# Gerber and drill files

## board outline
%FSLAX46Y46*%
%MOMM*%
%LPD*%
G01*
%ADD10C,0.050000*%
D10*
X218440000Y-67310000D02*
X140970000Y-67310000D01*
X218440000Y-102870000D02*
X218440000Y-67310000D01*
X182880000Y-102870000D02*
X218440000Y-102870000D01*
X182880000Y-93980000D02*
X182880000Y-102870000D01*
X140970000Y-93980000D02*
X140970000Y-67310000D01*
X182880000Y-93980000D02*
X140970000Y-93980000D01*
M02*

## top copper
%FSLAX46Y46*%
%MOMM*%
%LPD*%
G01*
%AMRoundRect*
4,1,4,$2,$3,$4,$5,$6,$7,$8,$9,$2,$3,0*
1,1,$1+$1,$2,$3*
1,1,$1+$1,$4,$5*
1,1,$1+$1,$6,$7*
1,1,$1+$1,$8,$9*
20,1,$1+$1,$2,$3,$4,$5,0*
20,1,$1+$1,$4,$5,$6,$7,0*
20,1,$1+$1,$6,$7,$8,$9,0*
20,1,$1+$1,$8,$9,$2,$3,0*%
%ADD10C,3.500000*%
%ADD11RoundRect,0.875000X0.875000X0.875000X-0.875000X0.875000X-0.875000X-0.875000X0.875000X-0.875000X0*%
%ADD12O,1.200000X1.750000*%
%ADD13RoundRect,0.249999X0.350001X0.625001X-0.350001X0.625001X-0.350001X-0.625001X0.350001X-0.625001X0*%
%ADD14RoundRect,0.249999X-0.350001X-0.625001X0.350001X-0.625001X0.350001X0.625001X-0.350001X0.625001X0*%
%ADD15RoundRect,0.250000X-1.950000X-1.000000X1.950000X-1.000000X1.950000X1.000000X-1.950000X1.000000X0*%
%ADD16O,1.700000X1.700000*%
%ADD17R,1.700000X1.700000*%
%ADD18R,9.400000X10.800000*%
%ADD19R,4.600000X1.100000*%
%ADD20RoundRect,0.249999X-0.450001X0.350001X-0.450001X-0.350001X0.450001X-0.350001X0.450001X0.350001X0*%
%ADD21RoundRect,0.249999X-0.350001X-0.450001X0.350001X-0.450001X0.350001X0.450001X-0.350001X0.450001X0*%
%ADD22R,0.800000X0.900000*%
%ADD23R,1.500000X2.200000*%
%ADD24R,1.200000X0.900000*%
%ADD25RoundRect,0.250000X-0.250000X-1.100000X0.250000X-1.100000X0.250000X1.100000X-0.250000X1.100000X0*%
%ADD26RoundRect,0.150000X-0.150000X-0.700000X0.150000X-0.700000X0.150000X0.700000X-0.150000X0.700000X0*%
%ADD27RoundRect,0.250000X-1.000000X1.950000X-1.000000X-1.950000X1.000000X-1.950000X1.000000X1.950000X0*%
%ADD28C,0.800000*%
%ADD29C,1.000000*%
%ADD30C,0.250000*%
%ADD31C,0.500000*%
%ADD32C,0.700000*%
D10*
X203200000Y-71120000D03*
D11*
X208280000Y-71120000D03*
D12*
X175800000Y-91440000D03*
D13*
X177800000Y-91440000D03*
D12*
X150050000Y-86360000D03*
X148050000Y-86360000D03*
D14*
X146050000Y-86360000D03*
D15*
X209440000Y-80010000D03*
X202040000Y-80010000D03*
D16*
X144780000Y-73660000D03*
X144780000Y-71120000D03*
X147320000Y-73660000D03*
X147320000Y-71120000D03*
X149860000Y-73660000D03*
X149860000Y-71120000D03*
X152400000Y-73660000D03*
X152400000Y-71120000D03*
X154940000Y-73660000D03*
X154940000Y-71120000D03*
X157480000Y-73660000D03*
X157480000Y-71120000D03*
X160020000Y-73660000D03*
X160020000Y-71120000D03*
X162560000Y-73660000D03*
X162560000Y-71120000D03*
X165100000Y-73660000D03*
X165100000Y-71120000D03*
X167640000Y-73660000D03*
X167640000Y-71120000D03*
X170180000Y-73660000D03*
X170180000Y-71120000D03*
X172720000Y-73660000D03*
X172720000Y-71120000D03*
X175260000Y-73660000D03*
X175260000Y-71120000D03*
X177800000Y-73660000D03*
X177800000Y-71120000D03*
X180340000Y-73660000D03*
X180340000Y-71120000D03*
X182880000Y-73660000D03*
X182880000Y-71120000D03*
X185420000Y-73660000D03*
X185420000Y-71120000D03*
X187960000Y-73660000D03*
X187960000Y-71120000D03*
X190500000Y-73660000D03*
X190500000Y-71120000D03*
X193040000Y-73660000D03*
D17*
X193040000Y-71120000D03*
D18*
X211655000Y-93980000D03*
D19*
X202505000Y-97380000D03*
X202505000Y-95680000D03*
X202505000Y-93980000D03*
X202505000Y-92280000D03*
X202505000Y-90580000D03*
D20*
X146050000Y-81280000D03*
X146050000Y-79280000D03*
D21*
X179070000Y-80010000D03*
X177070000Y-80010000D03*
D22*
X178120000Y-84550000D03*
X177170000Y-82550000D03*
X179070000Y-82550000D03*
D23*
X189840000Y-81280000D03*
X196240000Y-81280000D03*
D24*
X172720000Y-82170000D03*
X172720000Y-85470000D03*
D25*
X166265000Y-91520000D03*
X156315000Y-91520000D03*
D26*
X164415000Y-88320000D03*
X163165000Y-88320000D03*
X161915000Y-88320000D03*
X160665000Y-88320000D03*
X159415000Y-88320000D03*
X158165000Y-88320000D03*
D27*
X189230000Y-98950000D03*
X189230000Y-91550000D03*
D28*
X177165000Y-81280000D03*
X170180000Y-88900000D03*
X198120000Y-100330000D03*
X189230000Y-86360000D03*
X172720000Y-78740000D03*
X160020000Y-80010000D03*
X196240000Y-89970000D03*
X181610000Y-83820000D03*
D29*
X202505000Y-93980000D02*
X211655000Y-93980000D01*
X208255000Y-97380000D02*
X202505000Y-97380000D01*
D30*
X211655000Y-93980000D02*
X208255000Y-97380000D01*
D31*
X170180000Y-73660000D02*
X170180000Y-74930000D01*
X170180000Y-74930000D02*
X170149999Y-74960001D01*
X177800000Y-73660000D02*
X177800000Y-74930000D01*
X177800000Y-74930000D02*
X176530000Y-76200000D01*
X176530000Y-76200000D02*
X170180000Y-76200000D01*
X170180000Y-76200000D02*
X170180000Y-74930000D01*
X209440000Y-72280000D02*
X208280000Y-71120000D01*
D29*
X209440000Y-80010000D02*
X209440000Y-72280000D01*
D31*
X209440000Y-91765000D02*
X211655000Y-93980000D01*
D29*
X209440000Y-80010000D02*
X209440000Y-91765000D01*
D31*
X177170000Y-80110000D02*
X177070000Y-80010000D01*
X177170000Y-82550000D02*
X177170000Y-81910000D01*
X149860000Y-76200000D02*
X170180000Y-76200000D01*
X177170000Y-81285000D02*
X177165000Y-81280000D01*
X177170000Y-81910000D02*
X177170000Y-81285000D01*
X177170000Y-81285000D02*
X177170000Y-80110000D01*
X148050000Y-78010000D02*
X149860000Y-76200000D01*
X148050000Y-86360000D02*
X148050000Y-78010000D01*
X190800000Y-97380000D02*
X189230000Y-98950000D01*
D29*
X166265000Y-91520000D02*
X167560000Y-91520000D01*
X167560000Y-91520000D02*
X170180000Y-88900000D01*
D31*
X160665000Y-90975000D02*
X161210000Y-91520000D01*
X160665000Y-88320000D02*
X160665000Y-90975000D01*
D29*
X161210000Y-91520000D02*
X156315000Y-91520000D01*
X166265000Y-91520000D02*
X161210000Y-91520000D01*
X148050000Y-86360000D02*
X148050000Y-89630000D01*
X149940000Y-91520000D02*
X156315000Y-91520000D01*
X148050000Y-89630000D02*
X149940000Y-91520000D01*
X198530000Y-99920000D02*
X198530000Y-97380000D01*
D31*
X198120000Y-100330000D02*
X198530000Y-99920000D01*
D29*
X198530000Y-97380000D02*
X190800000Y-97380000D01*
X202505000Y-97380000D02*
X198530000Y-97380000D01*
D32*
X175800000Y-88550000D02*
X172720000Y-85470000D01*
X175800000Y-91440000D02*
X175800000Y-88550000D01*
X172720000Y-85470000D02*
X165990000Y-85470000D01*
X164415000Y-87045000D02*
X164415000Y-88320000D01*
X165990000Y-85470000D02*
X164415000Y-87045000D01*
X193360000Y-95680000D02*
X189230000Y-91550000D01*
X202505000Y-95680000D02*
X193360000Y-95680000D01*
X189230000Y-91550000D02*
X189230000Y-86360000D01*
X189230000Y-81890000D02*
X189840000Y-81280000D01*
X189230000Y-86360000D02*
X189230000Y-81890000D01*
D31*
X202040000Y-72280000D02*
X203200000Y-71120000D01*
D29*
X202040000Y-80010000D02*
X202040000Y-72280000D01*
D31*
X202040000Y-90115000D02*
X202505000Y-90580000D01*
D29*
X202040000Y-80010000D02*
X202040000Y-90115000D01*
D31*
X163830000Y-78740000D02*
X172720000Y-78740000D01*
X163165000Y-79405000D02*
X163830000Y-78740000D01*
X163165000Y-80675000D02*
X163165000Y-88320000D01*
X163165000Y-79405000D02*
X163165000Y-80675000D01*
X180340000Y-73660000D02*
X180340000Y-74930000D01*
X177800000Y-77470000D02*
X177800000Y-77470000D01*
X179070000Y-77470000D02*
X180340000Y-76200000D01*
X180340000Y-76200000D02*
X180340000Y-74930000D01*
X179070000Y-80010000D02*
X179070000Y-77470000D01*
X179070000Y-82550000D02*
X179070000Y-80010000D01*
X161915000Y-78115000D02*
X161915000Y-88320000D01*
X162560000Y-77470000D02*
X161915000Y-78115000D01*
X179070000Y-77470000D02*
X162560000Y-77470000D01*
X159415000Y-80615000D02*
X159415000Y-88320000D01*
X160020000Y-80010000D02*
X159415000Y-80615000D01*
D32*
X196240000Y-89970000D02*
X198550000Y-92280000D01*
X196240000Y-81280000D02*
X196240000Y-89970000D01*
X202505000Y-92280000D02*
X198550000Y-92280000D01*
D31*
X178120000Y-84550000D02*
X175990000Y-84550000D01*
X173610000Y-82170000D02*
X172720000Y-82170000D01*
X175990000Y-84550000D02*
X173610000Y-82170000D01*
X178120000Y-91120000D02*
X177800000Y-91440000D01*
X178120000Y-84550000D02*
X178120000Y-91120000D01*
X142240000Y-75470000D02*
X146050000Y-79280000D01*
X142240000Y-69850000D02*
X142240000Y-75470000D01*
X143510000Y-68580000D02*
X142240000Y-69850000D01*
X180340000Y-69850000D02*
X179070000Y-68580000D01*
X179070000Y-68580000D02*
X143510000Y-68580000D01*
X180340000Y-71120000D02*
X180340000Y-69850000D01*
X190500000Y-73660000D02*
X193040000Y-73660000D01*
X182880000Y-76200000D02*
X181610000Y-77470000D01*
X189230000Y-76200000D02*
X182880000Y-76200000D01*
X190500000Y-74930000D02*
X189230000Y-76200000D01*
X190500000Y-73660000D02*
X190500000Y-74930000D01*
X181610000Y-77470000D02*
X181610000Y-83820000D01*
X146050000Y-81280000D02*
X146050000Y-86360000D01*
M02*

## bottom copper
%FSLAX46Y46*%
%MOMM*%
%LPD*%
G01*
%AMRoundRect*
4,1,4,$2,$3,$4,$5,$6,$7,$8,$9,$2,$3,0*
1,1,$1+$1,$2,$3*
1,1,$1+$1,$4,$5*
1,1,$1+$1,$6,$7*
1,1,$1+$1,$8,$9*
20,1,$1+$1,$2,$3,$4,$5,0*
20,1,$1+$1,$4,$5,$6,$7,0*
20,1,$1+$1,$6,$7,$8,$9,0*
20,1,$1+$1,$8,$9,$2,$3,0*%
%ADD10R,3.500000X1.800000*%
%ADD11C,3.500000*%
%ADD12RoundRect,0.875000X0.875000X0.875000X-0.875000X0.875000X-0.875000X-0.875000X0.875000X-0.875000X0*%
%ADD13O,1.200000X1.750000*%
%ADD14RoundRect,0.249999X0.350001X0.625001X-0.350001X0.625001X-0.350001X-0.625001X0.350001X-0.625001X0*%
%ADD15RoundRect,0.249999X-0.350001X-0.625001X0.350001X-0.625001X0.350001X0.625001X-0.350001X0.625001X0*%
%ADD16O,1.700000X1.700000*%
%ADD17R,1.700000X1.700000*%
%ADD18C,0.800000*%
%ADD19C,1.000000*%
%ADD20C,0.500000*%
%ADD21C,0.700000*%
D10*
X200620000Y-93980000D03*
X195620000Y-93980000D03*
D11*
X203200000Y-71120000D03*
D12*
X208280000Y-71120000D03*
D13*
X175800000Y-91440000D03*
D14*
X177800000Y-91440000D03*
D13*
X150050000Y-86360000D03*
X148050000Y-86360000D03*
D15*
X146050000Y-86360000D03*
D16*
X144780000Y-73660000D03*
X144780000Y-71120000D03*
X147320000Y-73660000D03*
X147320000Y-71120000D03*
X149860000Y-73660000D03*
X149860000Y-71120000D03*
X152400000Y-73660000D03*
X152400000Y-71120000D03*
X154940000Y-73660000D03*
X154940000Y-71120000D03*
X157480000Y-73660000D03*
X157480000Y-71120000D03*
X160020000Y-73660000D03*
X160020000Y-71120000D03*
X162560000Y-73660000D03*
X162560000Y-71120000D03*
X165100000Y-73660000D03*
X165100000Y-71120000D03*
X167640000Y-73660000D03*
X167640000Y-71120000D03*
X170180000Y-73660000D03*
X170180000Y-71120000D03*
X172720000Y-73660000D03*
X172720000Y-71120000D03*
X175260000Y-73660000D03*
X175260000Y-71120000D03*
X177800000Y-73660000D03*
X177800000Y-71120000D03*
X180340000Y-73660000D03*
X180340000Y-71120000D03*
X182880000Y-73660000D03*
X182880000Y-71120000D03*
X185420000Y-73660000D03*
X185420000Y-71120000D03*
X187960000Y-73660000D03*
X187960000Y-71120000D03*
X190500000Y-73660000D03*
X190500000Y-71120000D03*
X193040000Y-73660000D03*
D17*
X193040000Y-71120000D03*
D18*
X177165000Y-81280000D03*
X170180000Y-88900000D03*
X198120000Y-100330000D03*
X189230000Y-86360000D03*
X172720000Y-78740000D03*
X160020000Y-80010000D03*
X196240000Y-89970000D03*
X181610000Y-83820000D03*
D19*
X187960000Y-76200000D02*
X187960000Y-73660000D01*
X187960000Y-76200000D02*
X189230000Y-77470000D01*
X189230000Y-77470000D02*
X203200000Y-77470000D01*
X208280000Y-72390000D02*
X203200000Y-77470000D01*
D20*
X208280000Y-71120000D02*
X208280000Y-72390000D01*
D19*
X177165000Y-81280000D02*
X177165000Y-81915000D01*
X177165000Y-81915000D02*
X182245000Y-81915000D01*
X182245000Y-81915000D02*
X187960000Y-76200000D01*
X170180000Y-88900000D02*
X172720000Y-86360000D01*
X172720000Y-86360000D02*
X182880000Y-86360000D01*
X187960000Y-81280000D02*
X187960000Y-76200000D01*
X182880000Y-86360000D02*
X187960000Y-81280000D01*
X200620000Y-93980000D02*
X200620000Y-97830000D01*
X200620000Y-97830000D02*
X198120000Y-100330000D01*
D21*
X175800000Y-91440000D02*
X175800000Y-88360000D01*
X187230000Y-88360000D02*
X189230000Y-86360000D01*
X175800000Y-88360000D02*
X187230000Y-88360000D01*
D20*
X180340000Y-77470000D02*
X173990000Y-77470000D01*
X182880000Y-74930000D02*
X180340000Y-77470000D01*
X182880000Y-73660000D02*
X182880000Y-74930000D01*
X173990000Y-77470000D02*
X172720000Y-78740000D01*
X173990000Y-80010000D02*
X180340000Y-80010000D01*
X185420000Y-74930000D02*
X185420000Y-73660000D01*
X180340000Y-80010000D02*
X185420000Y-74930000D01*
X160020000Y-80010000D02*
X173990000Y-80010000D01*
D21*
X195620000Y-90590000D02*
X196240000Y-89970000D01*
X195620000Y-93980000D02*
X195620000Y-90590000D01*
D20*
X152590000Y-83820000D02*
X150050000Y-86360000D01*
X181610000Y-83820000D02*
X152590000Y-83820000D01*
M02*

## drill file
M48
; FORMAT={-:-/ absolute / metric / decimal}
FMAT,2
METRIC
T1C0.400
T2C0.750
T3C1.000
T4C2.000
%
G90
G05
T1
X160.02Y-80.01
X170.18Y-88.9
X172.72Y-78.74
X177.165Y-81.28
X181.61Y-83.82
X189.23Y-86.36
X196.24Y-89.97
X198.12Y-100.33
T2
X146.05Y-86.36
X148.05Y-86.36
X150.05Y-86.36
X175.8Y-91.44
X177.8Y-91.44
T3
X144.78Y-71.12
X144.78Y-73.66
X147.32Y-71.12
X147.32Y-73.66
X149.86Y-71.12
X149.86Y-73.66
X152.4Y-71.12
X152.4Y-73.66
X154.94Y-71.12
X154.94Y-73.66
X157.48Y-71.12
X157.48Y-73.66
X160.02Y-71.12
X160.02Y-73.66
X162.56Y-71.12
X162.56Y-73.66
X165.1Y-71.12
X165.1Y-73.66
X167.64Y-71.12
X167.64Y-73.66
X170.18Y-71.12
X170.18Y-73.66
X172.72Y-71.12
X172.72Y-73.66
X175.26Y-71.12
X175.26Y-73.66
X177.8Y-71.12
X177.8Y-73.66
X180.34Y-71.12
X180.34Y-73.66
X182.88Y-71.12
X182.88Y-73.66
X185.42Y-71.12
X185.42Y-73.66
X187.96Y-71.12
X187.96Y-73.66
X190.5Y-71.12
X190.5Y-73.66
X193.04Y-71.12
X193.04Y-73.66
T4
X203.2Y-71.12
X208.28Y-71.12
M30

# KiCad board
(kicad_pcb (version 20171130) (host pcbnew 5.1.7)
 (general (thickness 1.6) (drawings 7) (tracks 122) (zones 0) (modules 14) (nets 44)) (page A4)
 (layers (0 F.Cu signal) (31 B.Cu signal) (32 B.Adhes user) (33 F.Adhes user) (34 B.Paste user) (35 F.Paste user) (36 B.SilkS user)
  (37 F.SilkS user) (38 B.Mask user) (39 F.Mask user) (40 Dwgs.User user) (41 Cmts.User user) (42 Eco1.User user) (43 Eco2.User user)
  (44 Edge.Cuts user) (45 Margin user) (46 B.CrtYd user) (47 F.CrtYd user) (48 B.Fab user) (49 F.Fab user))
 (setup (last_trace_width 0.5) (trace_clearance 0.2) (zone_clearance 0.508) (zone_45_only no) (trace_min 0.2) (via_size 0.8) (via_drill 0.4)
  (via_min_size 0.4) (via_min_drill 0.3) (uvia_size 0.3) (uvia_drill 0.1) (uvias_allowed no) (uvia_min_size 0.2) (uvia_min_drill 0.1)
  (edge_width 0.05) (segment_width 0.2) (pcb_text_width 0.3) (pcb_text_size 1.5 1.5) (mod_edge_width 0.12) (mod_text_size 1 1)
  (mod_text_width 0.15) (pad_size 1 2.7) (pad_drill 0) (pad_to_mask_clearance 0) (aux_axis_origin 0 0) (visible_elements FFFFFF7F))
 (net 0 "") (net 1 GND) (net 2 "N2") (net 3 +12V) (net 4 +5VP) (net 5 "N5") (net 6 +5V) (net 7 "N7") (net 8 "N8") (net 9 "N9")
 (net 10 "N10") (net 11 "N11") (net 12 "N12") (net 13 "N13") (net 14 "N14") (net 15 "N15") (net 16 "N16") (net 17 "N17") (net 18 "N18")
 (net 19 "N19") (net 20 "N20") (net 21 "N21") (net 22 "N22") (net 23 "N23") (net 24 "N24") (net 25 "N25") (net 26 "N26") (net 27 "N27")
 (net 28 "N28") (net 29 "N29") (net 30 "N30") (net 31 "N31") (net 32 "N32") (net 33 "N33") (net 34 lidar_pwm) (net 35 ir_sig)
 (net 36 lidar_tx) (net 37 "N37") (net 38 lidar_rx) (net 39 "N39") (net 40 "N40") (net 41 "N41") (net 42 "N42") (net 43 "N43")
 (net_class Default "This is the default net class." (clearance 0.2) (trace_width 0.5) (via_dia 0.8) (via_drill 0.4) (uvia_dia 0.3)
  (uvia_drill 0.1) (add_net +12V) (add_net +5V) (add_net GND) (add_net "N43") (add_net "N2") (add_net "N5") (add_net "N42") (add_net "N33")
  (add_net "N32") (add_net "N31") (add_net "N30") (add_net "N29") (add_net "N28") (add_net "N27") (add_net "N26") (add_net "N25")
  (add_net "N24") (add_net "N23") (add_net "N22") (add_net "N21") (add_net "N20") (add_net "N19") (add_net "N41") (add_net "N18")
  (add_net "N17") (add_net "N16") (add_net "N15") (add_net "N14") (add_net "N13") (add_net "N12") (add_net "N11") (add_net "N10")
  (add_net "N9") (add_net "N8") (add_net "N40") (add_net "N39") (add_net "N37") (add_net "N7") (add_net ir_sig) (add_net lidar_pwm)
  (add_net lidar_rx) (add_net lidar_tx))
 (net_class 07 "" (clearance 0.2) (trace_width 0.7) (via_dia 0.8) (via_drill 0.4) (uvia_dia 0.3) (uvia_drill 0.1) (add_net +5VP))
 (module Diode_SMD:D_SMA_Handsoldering (layer B.Cu) (at 198.12 93.98)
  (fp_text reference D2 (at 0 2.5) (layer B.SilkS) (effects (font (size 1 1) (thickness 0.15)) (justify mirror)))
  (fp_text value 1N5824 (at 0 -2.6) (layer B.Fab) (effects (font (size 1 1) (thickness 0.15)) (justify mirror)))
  (pad 2 smd rect (at 2.5 0) (size 3.5 1.8) (layers B.Cu B.Paste B.Mask) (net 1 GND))
  (pad 1 smd rect (at -2.5 0) (size 3.5 1.8) (layers B.Cu B.Paste B.Mask) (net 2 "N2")))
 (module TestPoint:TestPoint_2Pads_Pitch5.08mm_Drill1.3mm (layer F.Cu) (at 208.28 71.12 180)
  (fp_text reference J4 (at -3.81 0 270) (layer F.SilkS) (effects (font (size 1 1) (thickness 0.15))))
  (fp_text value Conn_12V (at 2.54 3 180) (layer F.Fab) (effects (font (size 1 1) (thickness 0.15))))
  (pad 2 thru_hole circle (at 5.08 0 180) (size 3.5 3.5) (drill 2) (layers *.Cu *.Mask) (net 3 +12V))
  (pad 1 thru_hole roundrect (at 0 0 180) (size 3.5 3.5) (drill 2) (layers *.Cu *.Mask) (roundrect_rratio 0.25) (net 1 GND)))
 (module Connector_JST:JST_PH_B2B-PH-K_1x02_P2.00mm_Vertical (layer F.Cu) (at 177.8 91.44 180)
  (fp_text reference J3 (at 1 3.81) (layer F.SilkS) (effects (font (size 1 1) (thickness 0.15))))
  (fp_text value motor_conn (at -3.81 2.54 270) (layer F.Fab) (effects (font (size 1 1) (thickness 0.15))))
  (pad 2 thru_hole oval (at 2 0 180) (size 1.2 1.75) (drill 0.75) (layers *.Cu *.Mask) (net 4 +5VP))
  (pad 1 thru_hole roundrect (at 0 0 180) (size 1.2 1.75) (drill 0.75) (layers *.Cu *.Mask) (roundrect_rratio 0.2083325) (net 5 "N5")))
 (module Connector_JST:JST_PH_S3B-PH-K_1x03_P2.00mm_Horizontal (layer F.Cu) (at 146.05 86.36)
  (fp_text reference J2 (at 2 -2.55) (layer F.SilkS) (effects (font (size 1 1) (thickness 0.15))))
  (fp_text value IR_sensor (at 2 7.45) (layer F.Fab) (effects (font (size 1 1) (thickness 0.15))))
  (pad 3 thru_hole oval (at 4 0) (size 1.2 1.75) (drill 0.75) (layers *.Cu *.Mask) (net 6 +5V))
  (pad 2 thru_hole oval (at 2 0) (size 1.2 1.75) (drill 0.75) (layers *.Cu *.Mask) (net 1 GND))
  (pad 1 thru_hole roundrect (at 0 0) (size 1.2 1.75) (drill 0.75) (layers *.Cu *.Mask) (roundrect_rratio 0.2083325) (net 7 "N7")))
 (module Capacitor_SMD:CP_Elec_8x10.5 (layer F.Cu) (at 205.74 80.01)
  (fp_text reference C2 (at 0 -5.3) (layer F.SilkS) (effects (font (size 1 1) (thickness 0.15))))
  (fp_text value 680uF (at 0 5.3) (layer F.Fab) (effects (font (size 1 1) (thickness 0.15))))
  (pad 2 smd roundrect (at 3.7 0) (size 4.4 2.5) (layers F.Cu F.Paste F.Mask) (roundrect_rratio 0.1) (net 1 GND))
  (pad 1 smd roundrect (at -3.7 0) (size 4.4 2.5) (layers F.Cu F.Paste F.Mask) (roundrect_rratio 0.1) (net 3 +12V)))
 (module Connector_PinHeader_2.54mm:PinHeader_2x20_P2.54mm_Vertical (layer F.Cu) (at 193.04 71.12 270)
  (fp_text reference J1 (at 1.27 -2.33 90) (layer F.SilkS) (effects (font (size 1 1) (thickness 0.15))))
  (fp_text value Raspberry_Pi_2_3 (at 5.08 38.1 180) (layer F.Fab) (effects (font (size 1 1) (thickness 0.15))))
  (pad 40 thru_hole oval (at 2.54 48.26 270) (size 1.7 1.7) (drill 1) (layers *.Cu *.Mask) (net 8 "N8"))
  (pad 39 thru_hole oval (at 0 48.26 270) (size 1.7 1.7) (drill 1) (layers *.Cu *.Mask) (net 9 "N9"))
  (pad 38 thru_hole oval (at 2.54 45.72 270) (size 1.7 1.7) (drill 1) (layers *.Cu *.Mask) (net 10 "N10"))
  (pad 37 thru_hole oval (at 0 45.72 270) (size 1.7 1.7) (drill 1) (layers *.Cu *.Mask) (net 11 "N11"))
  (pad 36 thru_hole oval (at 2.54 43.18 270) (size 1.7 1.7) (drill 1) (layers *.Cu *.Mask) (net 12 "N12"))
  (pad 35 thru_hole oval (at 0 43.18 270) (size 1.7 1.7) (drill 1) (layers *.Cu *.Mask) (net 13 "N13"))
  (pad 34 thru_hole oval (at 2.54 40.64 270) (size 1.7 1.7) (drill 1) (layers *.Cu *.Mask) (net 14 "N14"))
  (pad 33 thru_hole oval (at 0 40.64 270) (size 1.7 1.7) (drill 1) (layers *.Cu *.Mask) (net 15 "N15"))
  (pad 32 thru_hole oval (at 2.54 38.1 270) (size 1.7 1.7) (drill 1) (layers *.Cu *.Mask) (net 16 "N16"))
  (pad 31 thru_hole oval (at 0 38.1 270) (size 1.7 1.7) (drill 1) (layers *.Cu *.Mask) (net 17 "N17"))
  (pad 30 thru_hole oval (at 2.54 35.56 270) (size 1.7 1.7) (drill 1) (layers *.Cu *.Mask) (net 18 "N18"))
  (pad 29 thru_hole oval (at 0 35.56 270) (size 1.7 1.7) (drill 1) (layers *.Cu *.Mask) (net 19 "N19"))
  (pad 28 thru_hole oval (at 2.54 33.02 270) (size 1.7 1.7) (drill 1) (layers *.Cu *.Mask) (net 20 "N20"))
  (pad 27 thru_hole oval (at 0 33.02 270) (size 1.7 1.7) (drill 1) (layers *.Cu *.Mask) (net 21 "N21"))
  (pad 26 thru_hole oval (at 2.54 30.48 270) (size 1.7 1.7) (drill 1) (layers *.Cu *.Mask) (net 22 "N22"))
  (pad 25 thru_hole oval (at 0 30.48 270) (size 1.7 1.7) (drill 1) (layers *.Cu *.Mask) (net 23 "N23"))
  (pad 24 thru_hole oval (at 2.54 27.94 270) (size 1.7 1.7) (drill 1) (layers *.Cu *.Mask) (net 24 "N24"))
  (pad 23 thru_hole oval (at 0 27.94 270) (size 1.7 1.7) (drill 1) (layers *.Cu *.Mask) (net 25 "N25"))
  (pad 22 thru_hole oval (at 2.54 25.4 270) (size 1.7 1.7) (drill 1) (layers *.Cu *.Mask) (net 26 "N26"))
  (pad 21 thru_hole oval (at 0 25.4 270) (size 1.7 1.7) (drill 1) (layers *.Cu *.Mask) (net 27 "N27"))
  (pad 20 thru_hole oval (at 2.54 22.86 270) (size 1.7 1.7) (drill 1) (layers *.Cu *.Mask) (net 1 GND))
  (pad 19 thru_hole oval (at 0 22.86 270) (size 1.7 1.7) (drill 1) (layers *.Cu *.Mask) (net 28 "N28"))
  (pad 18 thru_hole oval (at 2.54 20.32 270) (size 1.7 1.7) (drill 1) (layers *.Cu *.Mask) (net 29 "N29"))
  (pad 17 thru_hole oval (at 0 20.32 270) (size 1.7 1.7) (drill 1) (layers *.Cu *.Mask) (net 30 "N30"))
  (pad 16 thru_hole oval (at 2.54 17.78 270) (size 1.7 1.7) (drill 1) (layers *.Cu *.Mask) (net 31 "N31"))
  (pad 15 thru_hole oval (at 0 17.78 270) (size 1.7 1.7) (drill 1) (layers *.Cu *.Mask) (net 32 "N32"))
  (pad 14 thru_hole oval (at 2.54 15.24 270) (size 1.7 1.7) (drill 1) (layers *.Cu *.Mask) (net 1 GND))
  (pad 13 thru_hole oval (at 0 15.24 270) (size 1.7 1.7) (drill 1) (layers *.Cu *.Mask) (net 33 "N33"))
  (pad 12 thru_hole oval (at 2.54 12.7 270) (size 1.7 1.7) (drill 1) (layers *.Cu *.Mask) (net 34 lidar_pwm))
  (pad 11 thru_hole oval (at 0 12.7 270) (size 1.7 1.7) (drill 1) (layers *.Cu *.Mask) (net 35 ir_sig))
  (pad 10 thru_hole oval (at 2.54 10.16 270) (size 1.7 1.7) (drill 1) (layers *.Cu *.Mask) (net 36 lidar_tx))
  (pad 9 thru_hole oval (at 0 10.16 270) (size 1.7 1.7) (drill 1) (layers *.Cu *.Mask) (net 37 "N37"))
  (pad 8 thru_hole oval (at 2.54 7.62 270) (size 1.7 1.7) (drill 1) (layers *.Cu *.Mask) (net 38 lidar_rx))
  (pad 7 thru_hole oval (at 0 7.62 270) (size 1.7 1.7) (drill 1) (layers *.Cu *.Mask) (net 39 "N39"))
  (pad 6 thru_hole oval (at 2.54 5.08 270) (size 1.7 1.7) (drill 1) (layers *.Cu *.Mask) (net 1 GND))
  (pad 5 thru_hole oval (at 0 5.08 270) (size 1.7 1.7) (drill 1) (layers *.Cu *.Mask) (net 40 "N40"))
  (pad 4 thru_hole oval (at 2.54 2.54 270) (size 1.7 1.7) (drill 1) (layers *.Cu *.Mask) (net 6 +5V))
  (pad 3 thru_hole oval (at 0 2.54 270) (size 1.7 1.7) (drill 1) (layers *.Cu *.Mask) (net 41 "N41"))
  (pad 2 thru_hole oval (at 2.54 0 270) (size 1.7 1.7) (drill 1) (layers *.Cu *.Mask) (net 6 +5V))
  (pad 1 thru_hole rect (at 0 0 270) (size 1.7 1.7) (drill 1) (layers *.Cu *.Mask) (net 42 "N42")))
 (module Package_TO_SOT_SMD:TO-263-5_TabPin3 (layer F.Cu) (at 208.28 93.98)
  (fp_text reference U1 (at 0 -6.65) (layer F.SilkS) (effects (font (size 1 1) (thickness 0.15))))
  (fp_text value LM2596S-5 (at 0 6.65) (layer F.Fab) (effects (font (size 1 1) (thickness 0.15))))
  (pad "" smd rect (at 0.95 2.775) (size 4.55 5.25) (layers F.Paste))
  (pad "" smd rect (at 5.8 -2.775) (size 4.55 5.25) (layers F.Paste))
  (pad "" smd rect (at 0.95 -2.775) (size 4.55 5.25) (layers F.Paste))
  (pad "" smd rect (at 5.8 2.775) (size 4.55 5.25) (layers F.Paste))
  (pad 3 smd rect (at 3.375 0) (size 9.4 10.8) (layers F.Cu F.Mask) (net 1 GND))
  (pad 5 smd rect (at -5.775 3.4) (size 4.6 1.1) (layers F.Cu F.Paste F.Mask) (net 1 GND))
  (pad 4 smd rect (at -5.775 1.7) (size 4.6 1.1) (layers F.Cu F.Paste F.Mask) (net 4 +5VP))
  (pad 3 smd rect (at -5.775 0) (size 4.6 1.1) (layers F.Cu F.Paste F.Mask) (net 1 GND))
  (pad 2 smd rect (at -5.775 -1.7) (size 4.6 1.1) (layers F.Cu F.Paste F.Mask) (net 2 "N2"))
  (pad 1 smd rect (at -5.775 -3.4) (size 4.6 1.1) (layers F.Cu F.Paste F.Mask) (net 3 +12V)))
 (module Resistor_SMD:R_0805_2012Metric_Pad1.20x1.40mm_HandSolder (layer F.Cu) (at 146.05 80.28 270)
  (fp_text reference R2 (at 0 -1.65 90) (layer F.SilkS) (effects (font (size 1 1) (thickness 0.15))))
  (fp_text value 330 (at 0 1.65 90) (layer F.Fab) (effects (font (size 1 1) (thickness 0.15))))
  (pad 2 smd roundrect (at 1 0 270) (size 1.2 1.4) (layers F.Cu F.Paste F.Mask) (roundrect_rratio 0.2083325) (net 7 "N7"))
  (pad 1 smd roundrect (at -1 0 270) (size 1.2 1.4) (layers F.Cu F.Paste F.Mask) (roundrect_rratio 0.2083325) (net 35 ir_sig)))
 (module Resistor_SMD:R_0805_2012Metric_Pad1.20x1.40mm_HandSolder (layer F.Cu) (at 178.07 80.01)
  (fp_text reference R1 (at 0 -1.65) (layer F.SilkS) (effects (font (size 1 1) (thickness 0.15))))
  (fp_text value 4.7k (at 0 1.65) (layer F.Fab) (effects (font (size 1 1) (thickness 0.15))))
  (pad 2 smd roundrect (at 1 0) (size 1.2 1.4) (layers F.Cu F.Paste F.Mask) (roundrect_rratio 0.2083325) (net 34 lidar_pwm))
  (pad 1 smd roundrect (at -1 0) (size 1.2 1.4) (layers F.Cu F.Paste F.Mask) (roundrect_rratio 0.2083325) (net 1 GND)))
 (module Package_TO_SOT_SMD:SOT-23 (layer F.Cu) (at 178.12 83.55 270)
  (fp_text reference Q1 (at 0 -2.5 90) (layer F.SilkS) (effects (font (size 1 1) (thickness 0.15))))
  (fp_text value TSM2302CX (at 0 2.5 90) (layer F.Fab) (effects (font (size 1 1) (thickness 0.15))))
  (pad 3 smd rect (at 1 0 270) (size 0.9 0.8) (layers F.Cu F.Paste F.Mask) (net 5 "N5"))
  (pad 2 smd rect (at -1 0.95 270) (size 0.9 0.8) (layers F.Cu F.Paste F.Mask) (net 1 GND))
  (pad 1 smd rect (at -1 -0.95 270) (size 0.9 0.8) (layers F.Cu F.Paste F.Mask) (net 34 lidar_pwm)))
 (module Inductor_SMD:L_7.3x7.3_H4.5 (layer F.Cu) (at 193.04 81.28 180)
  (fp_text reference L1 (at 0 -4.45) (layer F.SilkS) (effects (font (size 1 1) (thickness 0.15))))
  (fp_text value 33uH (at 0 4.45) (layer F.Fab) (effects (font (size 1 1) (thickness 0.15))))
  (pad 2 smd rect (at 3.2 0 180) (size 1.5 2.2) (layers F.Cu F.Paste F.Mask) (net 4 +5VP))
  (pad 1 smd rect (at -3.2 0 180) (size 1.5 2.2) (layers F.Cu F.Paste F.Mask) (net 2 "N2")))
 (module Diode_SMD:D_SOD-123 (layer F.Cu) (at 172.72 83.82 90)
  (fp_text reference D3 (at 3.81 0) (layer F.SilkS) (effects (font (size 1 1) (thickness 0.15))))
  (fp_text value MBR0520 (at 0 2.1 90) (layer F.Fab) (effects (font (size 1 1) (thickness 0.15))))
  (pad 2 smd rect (at 1.65 0 90) (size 0.9 1.2) (layers F.Cu F.Paste F.Mask) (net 5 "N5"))
  (pad 1 smd rect (at -1.65 0 90) (size 0.9 1.2) (layers F.Cu F.Paste F.Mask) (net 4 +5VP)))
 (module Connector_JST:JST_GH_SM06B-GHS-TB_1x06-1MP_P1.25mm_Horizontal (layer F.Cu) (at 161.29 90.17)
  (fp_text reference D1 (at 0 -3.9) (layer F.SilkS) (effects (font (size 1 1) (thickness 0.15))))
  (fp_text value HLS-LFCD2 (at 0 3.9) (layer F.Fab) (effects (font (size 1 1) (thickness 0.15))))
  (pad MP smd roundrect (at 4.975 1.35) (size 1 2.7) (layers F.Cu F.Paste F.Mask) (roundrect_rratio 0.25) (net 1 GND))
  (pad MP smd roundrect (at -4.975 1.35) (size 1 2.7) (layers F.Cu F.Paste F.Mask) (roundrect_rratio 0.25) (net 1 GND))
  (pad 6 smd roundrect (at 3.125 -1.85) (size 0.6 1.7) (layers F.Cu F.Paste F.Mask) (roundrect_rratio 0.25) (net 4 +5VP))
  (pad 5 smd roundrect (at 1.875 -1.85) (size 0.6 1.7) (layers F.Cu F.Paste F.Mask) (roundrect_rratio 0.25) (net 36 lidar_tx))
  (pad 4 smd roundrect (at 0.625 -1.85) (size 0.6 1.7) (layers F.Cu F.Paste F.Mask) (roundrect_rratio 0.25) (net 34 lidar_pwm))
  (pad 3 smd roundrect (at -0.625 -1.85) (size 0.6 1.7) (layers F.Cu F.Paste F.Mask) (roundrect_rratio 0.25) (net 1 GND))
  (pad 2 smd roundrect (at -1.875 -1.85) (size 0.6 1.7) (layers F.Cu F.Paste F.Mask) (roundrect_rratio 0.25) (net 38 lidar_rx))
  (pad 1 smd roundrect (at -3.125 -1.85) (size 0.6 1.7) (layers F.Cu F.Paste F.Mask) (roundrect_rratio 0.25) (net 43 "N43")))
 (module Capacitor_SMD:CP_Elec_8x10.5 (layer F.Cu) (at 189.23 95.25 270)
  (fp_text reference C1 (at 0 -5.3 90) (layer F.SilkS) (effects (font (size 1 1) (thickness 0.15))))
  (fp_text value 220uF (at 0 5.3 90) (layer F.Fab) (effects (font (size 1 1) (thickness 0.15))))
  (pad 2 smd roundrect (at 3.7 0 270) (size 4.4 2.5) (layers F.Cu F.Paste F.Mask) (roundrect_rratio 0.1) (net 1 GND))
  (pad 1 smd roundrect (at -3.7 0 270) (size 4.4 2.5) (layers F.Cu F.Paste F.Mask) (roundrect_rratio 0.1) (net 4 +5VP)))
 (gr_line (start 218.44 67.31) (end 140.97 67.31) (layer Edge.Cuts) (width 0.05))
 (gr_line (start 218.44 102.87) (end 218.44 67.31) (layer Edge.Cuts) (width 0.05))
 (gr_line (start 182.88 102.87) (end 218.44 102.87) (layer Edge.Cuts) (width 0.05))
 (gr_line (start 182.88 93.98) (end 182.88 102.87) (layer Edge.Cuts) (width 0.05))
 (gr_line (start 140.97 93.98) (end 140.97 67.31) (layer Edge.Cuts) (width 0.05))
 (gr_line (start 182.88 93.98) (end 140.97 93.98) (layer Edge.Cuts) (width 0.05))
 (segment (start 202.505 93.98) (end 211.655 93.98) (width 1) (layer F.Cu) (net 1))
 (segment (start 208.255 97.38) (end 202.505 97.38) (width 1) (layer F.Cu) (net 1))
 (segment (start 211.655 93.98) (end 208.255 97.38) (width 0.25) (layer F.Cu) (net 1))
 (segment (start 187.96 76.2) (end 187.96 73.66) (width 1) (layer B.Cu) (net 1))
 (segment (start 187.96 76.2) (end 189.23 77.47) (width 1) (layer B.Cu) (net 1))
 (segment (start 189.23 77.47) (end 203.2 77.47) (width 1) (layer B.Cu) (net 1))
 (segment (start 208.28 72.39) (end 203.2 77.47) (width 1) (layer B.Cu) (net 1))
 (segment (start 208.28 71.12) (end 208.28 72.39) (width 0.5) (layer B.Cu) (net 1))
 (segment (start 170.18 73.66) (end 170.18 74.93) (width 0.5) (layer F.Cu) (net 1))
 (segment (start 170.18 74.93) (end 170.149999 74.960001) (width 0.5) (layer F.Cu) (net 1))
 (segment (start 177.8 73.66) (end 177.8 74.93) (width 0.5) (layer F.Cu) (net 1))
 (segment (start 177.8 74.93) (end 176.53 76.2) (width 0.5) (layer F.Cu) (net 1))
 (segment (start 176.53 76.2) (end 170.18 76.2) (width 0.5) (layer F.Cu) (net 1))
 (segment (start 170.18 76.2) (end 170.18 74.93) (width 0.5) (layer F.Cu) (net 1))
 (segment (start 209.44 72.28) (end 208.28 71.12) (width 0.5) (layer F.Cu) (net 1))
 (segment (start 209.44 80.01) (end 209.44 72.28) (width 1) (layer F.Cu) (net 1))
 (segment (start 209.44 91.765) (end 211.655 93.98) (width 0.5) (layer F.Cu) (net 1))
 (segment (start 209.44 80.01) (end 209.44 91.765) (width 1) (layer F.Cu) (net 1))
 (segment (start 177.17 80.11) (end 177.07 80.01) (width 0.5) (layer F.Cu) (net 1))
 (segment (start 177.17 82.55) (end 177.17 81.91) (width 0.5) (layer F.Cu) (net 1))
 (segment (start 149.86 76.2) (end 170.18 76.2) (width 0.5) (layer F.Cu) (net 1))
 (via (at 177.165 81.28) (size 0.8) (drill 0.4) (layers F.Cu B.Cu) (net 1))
 (segment (start 177.17 81.285) (end 177.165 81.28) (width 0.5) (layer F.Cu) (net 1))
 (segment (start 177.17 81.91) (end 177.17 81.285) (width 0.5) (layer F.Cu) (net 1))
 (segment (start 177.17 81.285) (end 177.17 80.11) (width 0.5) (layer F.Cu) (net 1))
 (segment (start 177.165 81.28) (end 177.165 81.915) (width 1) (layer B.Cu) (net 1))
 (segment (start 177.165 81.915) (end 182.245 81.915) (width 1) (layer B.Cu) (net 1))
 (segment (start 182.245 81.915) (end 187.96 76.2) (width 1) (layer B.Cu) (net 1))
 (segment (start 148.05 78.01) (end 149.86 76.2) (width 0.5) (layer F.Cu) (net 1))
 (segment (start 148.05 86.36) (end 148.05 78.01) (width 0.5) (layer F.Cu) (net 1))
 (segment (start 190.8 97.38) (end 189.23 98.95) (width 0.5) (layer F.Cu) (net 1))
 (segment (start 166.265 91.52) (end 167.56 91.52) (width 1) (layer F.Cu) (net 1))
 (via (at 170.18 88.9) (size 0.8) (drill 0.4) (layers F.Cu B.Cu) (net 1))
 (segment (start 167.56 91.52) (end 170.18 88.9) (width 1) (layer F.Cu) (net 1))
 (segment (start 170.18 88.9) (end 172.72 86.36) (width 1) (layer B.Cu) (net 1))
 (segment (start 172.72 86.36) (end 182.88 86.36) (width 1) (layer B.Cu) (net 1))
 (segment (start 187.96 81.28) (end 187.96 76.2) (width 1) (layer B.Cu) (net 1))
 (segment (start 182.88 86.36) (end 187.96 81.28) (width 1) (layer B.Cu) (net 1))
 (segment (start 160.665 90.975) (end 161.21 91.52) (width 0.5) (layer F.Cu) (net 1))
 (segment (start 160.665 88.32) (end 160.665 90.975) (width 0.5) (layer F.Cu) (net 1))
 (segment (start 161.21 91.52) (end 156.315 91.52) (width 1) (layer F.Cu) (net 1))
 (segment (start 166.265 91.52) (end 161.21 91.52) (width 1) (layer F.Cu) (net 1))
 (segment (start 148.05 86.36) (end 148.05 89.63) (width 1) (layer F.Cu) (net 1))
 (segment (start 149.94 91.52) (end 156.315 91.52) (width 1) (layer F.Cu) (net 1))
 (segment (start 148.05 89.63) (end 149.94 91.52) (width 1) (layer F.Cu) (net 1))
 (segment (start 200.62 93.98) (end 200.62 97.83) (width 1) (layer B.Cu) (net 1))
 (via (at 198.12 100.33) (size 0.8) (drill 0.4) (layers F.Cu B.Cu) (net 1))
 (segment (start 200.62 97.83) (end 198.12 100.33) (width 1) (layer B.Cu) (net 1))
 (segment (start 198.53 99.92) (end 198.53 97.38) (width 1) (layer F.Cu) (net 1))
 (segment (start 198.12 100.33) (end 198.53 99.92) (width 0.5) (layer F.Cu) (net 1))
 (segment (start 198.53 97.38) (end 190.8 97.38) (width 1) (layer F.Cu) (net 1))
 (segment (start 202.505 97.38) (end 198.53 97.38) (width 1) (layer F.Cu) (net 1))
 (segment (start 175.8 88.55) (end 172.72 85.47) (width 0.7) (layer F.Cu) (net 4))
 (segment (start 175.8 91.44) (end 175.8 88.55) (width 0.7) (layer F.Cu) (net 4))
 (segment (start 175.8 91.44) (end 175.8 88.36) (width 0.7) (layer B.Cu) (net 4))
 (segment (start 172.72 85.47) (end 165.99 85.47) (width 0.7) (layer F.Cu) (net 4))
 (segment (start 164.415 87.045) (end 164.415 88.32) (width 0.7) (layer F.Cu) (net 4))
 (segment (start 165.99 85.47) (end 164.415 87.045) (width 0.7) (layer F.Cu) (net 4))
 (segment (start 193.36 95.68) (end 189.23 91.55) (width 0.7) (layer F.Cu) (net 4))
 (segment (start 202.505 95.68) (end 193.36 95.68) (width 0.7) (layer F.Cu) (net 4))
 (via (at 189.23 86.36) (size 0.8) (drill 0.4) (layers F.Cu B.Cu) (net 4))
 (segment (start 189.23 91.55) (end 189.23 86.36) (width 0.7) (layer F.Cu) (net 4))
 (segment (start 189.23 81.89) (end 189.84 81.28) (width 0.7) (layer F.Cu) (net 4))
 (segment (start 189.23 86.36) (end 189.23 81.89) (width 0.7) (layer F.Cu) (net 4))
 (segment (start 187.23 88.36) (end 189.23 86.36) (width 0.7) (layer B.Cu) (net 4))
 (segment (start 175.8 88.36) (end 187.23 88.36) (width 0.7) (layer B.Cu) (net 4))
 (segment (start 202.04 72.28) (end 203.2 71.12) (width 0.5) (layer F.Cu) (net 3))
 (segment (start 202.04 80.01) (end 202.04 72.28) (width 1) (layer F.Cu) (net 3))
 (segment (start 202.04 90.115) (end 202.505 90.58) (width 0.5) (layer F.Cu) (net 3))
 (segment (start 202.04 80.01) (end 202.04 90.115) (width 1) (layer F.Cu) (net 3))
 (segment (start 180.34 77.47) (end 173.99 77.47) (width 0.5) (layer B.Cu) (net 36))
 (segment (start 182.88 74.93) (end 180.34 77.47) (width 0.5) (layer B.Cu) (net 36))
 (segment (start 182.88 73.66) (end 182.88 74.93) (width 0.5) (layer B.Cu) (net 36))
 (via (at 172.72 78.74) (size 0.8) (drill 0.4) (layers F.Cu B.Cu) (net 36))
 (segment (start 163.83 78.74) (end 172.72 78.74) (width 0.5) (layer F.Cu) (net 36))
 (segment (start 163.165 79.405) (end 163.83 78.74) (width 0.5) (layer F.Cu) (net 36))
 (segment (start 173.99 77.47) (end 172.72 78.74) (width 0.5) (layer B.Cu) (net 36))
 (segment (start 163.165 80.675) (end 163.165 88.32) (width 0.5) (layer F.Cu) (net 36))
 (segment (start 163.165 79.405) (end 163.165 80.675) (width 0.5) (layer F.Cu) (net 36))
 (segment (start 180.34 73.66) (end 180.34 74.93) (width 0.5) (layer F.Cu) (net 34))
 (segment (start 177.8 77.47) (end 177.8 77.47) (width 0.5) (layer F.Cu) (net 34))
 (segment (start 179.07 77.47) (end 180.34 76.2) (width 0.5) (layer F.Cu) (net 34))
 (segment (start 180.34 76.2) (end 180.34 74.93) (width 0.5) (layer F.Cu) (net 34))
 (segment (start 179.07 80.01) (end 179.07 77.47) (width 0.5) (layer F.Cu) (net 34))
 (segment (start 179.07 82.55) (end 179.07 80.01) (width 0.5) (layer F.Cu) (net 34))
 (segment (start 161.915 78.115) (end 161.915 88.32) (width 0.5) (layer F.Cu) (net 34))
 (segment (start 162.56 77.47) (end 161.915 78.115) (width 0.5) (layer F.Cu) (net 34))
 (segment (start 179.07 77.47) (end 162.56 77.47) (width 0.5) (layer F.Cu) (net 34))
 (segment (start 173.99 80.01) (end 180.34 80.01) (width 0.5) (layer B.Cu) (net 38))
 (segment (start 185.42 74.93) (end 185.42 73.66) (width 0.5) (layer B.Cu) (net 38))
 (segment (start 180.34 80.01) (end 185.42 74.93) (width 0.5) (layer B.Cu) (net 38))
 (via (at 160.02 80.01) (size 0.8) (drill 0.4) (layers F.Cu B.Cu) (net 38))
 (segment (start 160.02 80.01) (end 173.99 80.01) (width 0.5) (layer B.Cu) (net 38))
 (segment (start 159.415 80.615) (end 159.415 88.32) (width 0.5) (layer F.Cu) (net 38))
 (segment (start 160.02 80.01) (end 159.415 80.615) (width 0.5) (layer F.Cu) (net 38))
 (segment (start 196.24 89.97) (end 198.55 92.28) (width 0.7) (layer F.Cu) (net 2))
 (segment (start 196.24 81.28) (end 196.24 89.97) (width 0.7) (layer F.Cu) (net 2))
 (segment (start 202.505 92.28) (end 198.55 92.28) (width 0.7) (layer F.Cu) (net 2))
 (via (at 196.24 89.97) (size 0.8) (drill 0.4) (layers F.Cu B.Cu) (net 2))
 (segment (start 195.62 90.59) (end 196.24 89.97) (width 0.7) (layer B.Cu) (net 2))
 (segment (start 195.62 93.98) (end 195.62 90.59) (width 0.7) (layer B.Cu) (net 2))
 (segment (start 178.12 84.55) (end 175.99 84.55) (width 0.5) (layer F.Cu) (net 5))
 (segment (start 173.61 82.17) (end 172.72 82.17) (width 0.5) (layer F.Cu) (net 5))
 (segment (start 175.99 84.55) (end 173.61 82.17) (width 0.5) (layer F.Cu) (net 5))
 (segment (start 178.12 91.12) (end 177.8 91.44) (width 0.5) (layer F.Cu) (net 5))
 (segment (start 178.12 84.55) (end 178.12 91.12) (width 0.5) (layer F.Cu) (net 5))
 (segment (start 142.24 75.47) (end 146.05 79.28) (width 0.5) (layer F.Cu) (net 35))
 (segment (start 142.24 69.85) (end 142.24 75.47) (width 0.5) (layer F.Cu) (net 35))
 (segment (start 143.51 68.58) (end 142.24 69.85) (width 0.5) (layer F.Cu) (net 35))
 (segment (start 180.34 69.85) (end 179.07 68.58) (width 0.5) (layer F.Cu) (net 35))
 (segment (start 179.07 68.58) (end 143.51 68.58) (width 0.5) (layer F.Cu) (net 35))
 (segment (start 180.34 71.12) (end 180.34 69.85) (width 0.5) (layer F.Cu) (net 35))
 (segment (start 190.5 73.66) (end 193.04 73.66) (width 0.5) (layer F.Cu) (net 6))
 (segment (start 182.88 76.2) (end 181.61 77.47) (width 0.5) (layer F.Cu) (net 6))
 (segment (start 189.23 76.2) (end 182.88 76.2) (width 0.5) (layer F.Cu) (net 6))
 (segment (start 190.5 74.93) (end 189.23 76.2) (width 0.5) (layer F.Cu) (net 6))
 (segment (start 190.5 73.66) (end 190.5 74.93) (width 0.5) (layer F.Cu) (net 6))
 (via (at 181.61 83.82) (size 0.8) (drill 0.4) (layers F.Cu B.Cu) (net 6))
 (segment (start 181.61 77.47) (end 181.61 83.82) (width 0.5) (layer F.Cu) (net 6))
 (segment (start 152.59 83.82) (end 150.05 86.36) (width 0.5) (layer B.Cu) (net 6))
 (segment (start 181.61 83.82) (end 152.59 83.82) (width 0.5) (layer B.Cu) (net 6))
 (segment (start 146.05 81.28) (end 146.05 86.36) (width 0.5) (layer F.Cu) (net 7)))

